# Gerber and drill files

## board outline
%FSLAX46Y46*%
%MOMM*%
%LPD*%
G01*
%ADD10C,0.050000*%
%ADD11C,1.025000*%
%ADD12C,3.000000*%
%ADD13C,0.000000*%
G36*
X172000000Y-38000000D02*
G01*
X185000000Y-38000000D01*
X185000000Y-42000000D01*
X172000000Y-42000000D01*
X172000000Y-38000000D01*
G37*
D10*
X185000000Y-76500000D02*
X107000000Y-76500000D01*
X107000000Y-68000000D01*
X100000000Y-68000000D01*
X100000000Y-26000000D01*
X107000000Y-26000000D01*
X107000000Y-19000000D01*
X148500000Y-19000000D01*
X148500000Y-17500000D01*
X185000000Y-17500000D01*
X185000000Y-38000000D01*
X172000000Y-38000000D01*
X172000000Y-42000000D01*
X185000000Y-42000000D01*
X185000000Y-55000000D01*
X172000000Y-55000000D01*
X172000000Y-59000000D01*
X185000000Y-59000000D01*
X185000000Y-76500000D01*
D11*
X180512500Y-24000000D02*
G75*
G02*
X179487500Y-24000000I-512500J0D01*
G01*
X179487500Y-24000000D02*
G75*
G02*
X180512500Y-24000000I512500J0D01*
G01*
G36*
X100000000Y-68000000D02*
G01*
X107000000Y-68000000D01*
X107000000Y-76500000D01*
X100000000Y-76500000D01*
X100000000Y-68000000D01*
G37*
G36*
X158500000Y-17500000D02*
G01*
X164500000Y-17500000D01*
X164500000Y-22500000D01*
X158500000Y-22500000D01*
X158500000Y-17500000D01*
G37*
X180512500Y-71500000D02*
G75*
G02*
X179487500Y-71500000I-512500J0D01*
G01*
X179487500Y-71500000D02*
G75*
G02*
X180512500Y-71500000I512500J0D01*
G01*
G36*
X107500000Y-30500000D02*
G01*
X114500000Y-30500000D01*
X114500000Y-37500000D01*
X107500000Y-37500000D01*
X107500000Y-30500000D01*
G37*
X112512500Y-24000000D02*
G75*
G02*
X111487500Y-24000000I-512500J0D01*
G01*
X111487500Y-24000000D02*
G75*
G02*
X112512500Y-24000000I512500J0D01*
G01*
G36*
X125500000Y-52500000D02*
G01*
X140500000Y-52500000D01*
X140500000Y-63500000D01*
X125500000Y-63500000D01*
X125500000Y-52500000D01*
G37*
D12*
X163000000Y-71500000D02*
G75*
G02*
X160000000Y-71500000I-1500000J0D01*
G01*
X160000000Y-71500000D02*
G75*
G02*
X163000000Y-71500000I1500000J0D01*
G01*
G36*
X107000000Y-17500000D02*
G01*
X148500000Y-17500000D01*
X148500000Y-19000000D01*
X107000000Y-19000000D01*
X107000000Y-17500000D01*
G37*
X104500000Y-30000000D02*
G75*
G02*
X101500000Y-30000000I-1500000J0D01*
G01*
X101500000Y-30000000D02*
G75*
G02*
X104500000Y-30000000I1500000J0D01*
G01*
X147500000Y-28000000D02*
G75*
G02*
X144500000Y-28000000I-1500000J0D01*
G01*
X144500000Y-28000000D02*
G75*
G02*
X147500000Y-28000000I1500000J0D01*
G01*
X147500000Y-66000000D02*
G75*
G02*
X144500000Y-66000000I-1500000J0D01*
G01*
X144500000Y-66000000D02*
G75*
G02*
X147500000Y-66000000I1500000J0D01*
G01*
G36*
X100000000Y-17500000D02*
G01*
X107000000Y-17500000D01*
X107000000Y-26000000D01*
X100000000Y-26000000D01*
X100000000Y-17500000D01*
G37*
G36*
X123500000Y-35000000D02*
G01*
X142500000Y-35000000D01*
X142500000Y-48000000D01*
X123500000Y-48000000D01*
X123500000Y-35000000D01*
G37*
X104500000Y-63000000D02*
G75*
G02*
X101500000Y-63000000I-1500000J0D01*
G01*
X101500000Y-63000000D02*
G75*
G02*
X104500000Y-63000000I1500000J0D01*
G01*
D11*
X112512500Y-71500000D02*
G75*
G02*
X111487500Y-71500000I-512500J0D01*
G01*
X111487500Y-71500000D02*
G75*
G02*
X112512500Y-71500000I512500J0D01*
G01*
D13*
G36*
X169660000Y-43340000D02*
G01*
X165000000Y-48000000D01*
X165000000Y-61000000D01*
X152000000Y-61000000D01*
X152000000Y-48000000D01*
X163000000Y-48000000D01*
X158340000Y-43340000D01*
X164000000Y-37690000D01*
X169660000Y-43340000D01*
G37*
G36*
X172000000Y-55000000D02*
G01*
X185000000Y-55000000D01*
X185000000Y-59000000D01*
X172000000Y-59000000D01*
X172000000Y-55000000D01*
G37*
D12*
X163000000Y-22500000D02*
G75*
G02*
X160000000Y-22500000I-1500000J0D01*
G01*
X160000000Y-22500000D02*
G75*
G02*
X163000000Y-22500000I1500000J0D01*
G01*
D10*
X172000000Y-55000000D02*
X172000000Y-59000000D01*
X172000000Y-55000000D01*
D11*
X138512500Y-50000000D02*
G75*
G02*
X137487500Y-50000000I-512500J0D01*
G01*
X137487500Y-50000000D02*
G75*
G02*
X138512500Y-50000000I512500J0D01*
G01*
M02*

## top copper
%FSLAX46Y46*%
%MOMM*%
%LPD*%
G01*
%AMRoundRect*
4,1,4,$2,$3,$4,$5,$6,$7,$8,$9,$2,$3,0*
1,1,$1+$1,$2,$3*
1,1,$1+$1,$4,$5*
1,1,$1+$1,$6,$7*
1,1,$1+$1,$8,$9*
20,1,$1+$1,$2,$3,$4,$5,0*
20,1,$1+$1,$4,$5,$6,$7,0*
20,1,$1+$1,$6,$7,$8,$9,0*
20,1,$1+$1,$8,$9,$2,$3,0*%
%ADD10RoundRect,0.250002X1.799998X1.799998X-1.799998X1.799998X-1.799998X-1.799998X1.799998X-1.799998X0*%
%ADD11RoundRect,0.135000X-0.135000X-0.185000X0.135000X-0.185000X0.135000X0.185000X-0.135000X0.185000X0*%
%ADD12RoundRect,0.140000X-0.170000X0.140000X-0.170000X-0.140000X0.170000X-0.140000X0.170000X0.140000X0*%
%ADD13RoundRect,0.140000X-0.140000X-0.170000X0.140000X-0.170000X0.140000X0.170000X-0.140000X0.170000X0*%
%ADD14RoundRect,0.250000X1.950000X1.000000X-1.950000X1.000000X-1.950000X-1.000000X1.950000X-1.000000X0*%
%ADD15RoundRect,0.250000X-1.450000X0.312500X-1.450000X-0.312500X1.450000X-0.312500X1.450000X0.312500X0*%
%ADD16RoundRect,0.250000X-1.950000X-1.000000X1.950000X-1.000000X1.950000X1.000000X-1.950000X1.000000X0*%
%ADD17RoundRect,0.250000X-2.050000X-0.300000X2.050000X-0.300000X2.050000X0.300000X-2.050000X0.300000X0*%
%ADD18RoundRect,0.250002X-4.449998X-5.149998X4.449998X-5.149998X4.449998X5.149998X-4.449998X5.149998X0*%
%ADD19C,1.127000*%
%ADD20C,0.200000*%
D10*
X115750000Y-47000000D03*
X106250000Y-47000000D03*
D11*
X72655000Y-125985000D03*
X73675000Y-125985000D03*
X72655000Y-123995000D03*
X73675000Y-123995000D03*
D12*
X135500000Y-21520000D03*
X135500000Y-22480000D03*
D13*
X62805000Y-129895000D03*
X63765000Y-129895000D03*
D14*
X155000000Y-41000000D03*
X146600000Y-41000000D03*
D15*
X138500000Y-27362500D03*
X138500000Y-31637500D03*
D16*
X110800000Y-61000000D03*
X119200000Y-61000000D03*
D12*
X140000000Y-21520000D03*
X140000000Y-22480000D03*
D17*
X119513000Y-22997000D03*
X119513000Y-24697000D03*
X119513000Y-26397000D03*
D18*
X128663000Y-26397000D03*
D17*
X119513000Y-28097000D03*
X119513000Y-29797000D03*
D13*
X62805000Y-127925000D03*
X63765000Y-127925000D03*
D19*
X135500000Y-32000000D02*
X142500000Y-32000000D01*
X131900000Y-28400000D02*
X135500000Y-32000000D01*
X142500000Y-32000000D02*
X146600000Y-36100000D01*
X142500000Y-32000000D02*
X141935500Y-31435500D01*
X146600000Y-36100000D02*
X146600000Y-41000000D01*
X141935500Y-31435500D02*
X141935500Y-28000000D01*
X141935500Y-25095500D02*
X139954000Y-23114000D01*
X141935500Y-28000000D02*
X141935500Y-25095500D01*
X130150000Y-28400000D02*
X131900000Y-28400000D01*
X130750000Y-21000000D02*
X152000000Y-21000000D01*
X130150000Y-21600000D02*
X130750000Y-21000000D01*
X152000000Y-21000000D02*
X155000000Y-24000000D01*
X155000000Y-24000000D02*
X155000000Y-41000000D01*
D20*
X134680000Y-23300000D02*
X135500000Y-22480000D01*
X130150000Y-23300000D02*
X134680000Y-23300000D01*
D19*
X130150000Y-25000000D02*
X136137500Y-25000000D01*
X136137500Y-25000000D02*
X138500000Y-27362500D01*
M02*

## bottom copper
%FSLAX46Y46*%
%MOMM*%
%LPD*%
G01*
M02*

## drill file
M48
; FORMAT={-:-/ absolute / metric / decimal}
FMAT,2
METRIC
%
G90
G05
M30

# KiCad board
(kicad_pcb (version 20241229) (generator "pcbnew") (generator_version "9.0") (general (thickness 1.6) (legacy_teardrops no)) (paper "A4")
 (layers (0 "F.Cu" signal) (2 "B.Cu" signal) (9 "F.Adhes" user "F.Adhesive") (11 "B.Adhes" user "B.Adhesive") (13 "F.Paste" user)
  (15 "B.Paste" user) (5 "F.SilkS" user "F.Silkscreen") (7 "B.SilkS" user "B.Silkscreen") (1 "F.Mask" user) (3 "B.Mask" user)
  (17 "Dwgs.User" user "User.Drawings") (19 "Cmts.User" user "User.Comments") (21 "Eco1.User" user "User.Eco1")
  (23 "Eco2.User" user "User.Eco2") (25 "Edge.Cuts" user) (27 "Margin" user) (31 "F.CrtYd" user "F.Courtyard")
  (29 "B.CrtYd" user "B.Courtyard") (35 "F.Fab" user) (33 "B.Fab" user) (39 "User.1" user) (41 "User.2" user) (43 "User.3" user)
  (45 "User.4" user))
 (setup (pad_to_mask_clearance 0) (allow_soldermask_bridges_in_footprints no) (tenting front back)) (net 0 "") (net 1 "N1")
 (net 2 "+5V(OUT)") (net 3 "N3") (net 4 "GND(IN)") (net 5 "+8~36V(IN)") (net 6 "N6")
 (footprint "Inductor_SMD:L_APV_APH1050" (layer "F.Cu") (at 111 47 180)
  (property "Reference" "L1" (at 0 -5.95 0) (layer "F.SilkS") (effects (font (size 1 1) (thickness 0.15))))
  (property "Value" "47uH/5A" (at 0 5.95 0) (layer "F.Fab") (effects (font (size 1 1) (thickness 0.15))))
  (pad "1" smd roundrect (at -4.75 0 180) (size 4.1 4.1) (layers "F.Cu" "F.Mask" "F.Paste") (roundrect_rratio 0.060976) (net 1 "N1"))
  (pad "2" smd roundrect (at 4.75 0 180) (size 4.1 4.1) (layers "F.Cu" "F.Mask" "F.Paste") (roundrect_rratio 0.060976) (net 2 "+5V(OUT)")))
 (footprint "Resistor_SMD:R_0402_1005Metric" (layer "F.Cu") (at 73.165 125.985)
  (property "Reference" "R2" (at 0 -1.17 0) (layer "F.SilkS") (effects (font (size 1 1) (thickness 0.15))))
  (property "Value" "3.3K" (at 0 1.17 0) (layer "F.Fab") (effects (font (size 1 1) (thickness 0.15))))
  (pad "1" smd roundrect (at -0.51 0) (size 0.54 0.64) (layers "F.Cu" "F.Mask" "F.Paste") (roundrect_rratio 0.25) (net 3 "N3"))
  (pad "2" smd roundrect (at 0.51 0) (size 0.54 0.64) (layers "F.Cu" "F.Mask" "F.Paste") (roundrect_rratio 0.25) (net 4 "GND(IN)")))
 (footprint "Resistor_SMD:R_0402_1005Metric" (layer "F.Cu") (at 73.165 123.995)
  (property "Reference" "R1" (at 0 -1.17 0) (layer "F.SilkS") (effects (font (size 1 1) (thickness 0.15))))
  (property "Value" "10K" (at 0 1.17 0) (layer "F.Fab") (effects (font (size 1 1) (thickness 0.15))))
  (pad "1" smd roundrect (at -0.51 0) (size 0.54 0.64) (layers "F.Cu" "F.Mask" "F.Paste") (roundrect_rratio 0.25) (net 2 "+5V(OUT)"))
  (pad "2" smd roundrect (at 0.51 0) (size 0.54 0.64) (layers "F.Cu" "F.Mask" "F.Paste") (roundrect_rratio 0.25) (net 3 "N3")))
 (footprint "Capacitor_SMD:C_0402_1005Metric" (layer "F.Cu") (at 135.5 22 -90)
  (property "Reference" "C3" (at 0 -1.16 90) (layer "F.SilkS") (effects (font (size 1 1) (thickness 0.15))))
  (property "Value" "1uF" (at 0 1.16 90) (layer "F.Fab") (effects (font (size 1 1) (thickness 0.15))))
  (pad "1" smd roundrect (at -0.48 0 270) (size 0.56 0.62) (layers "F.Cu" "F.Mask" "F.Paste") (roundrect_rratio 0.25) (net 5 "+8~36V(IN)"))
  (pad "2" smd roundrect (at 0.48 0 270) (size 0.56 0.62) (layers "F.Cu" "F.Mask" "F.Paste") (roundrect_rratio 0.25) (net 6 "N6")))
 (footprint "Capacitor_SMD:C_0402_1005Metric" (layer "F.Cu") (at 63.285 129.895)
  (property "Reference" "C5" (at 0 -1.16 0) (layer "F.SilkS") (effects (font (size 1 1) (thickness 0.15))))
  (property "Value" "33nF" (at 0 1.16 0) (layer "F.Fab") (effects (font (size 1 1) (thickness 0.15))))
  (pad "1" smd roundrect (at -0.48 0) (size 0.56 0.62) (layers "F.Cu" "F.Mask" "F.Paste") (roundrect_rratio 0.25) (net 2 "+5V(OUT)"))
  (pad "2" smd roundrect (at 0.48 0) (size 0.56 0.62) (layers "F.Cu" "F.Mask" "F.Paste") (roundrect_rratio 0.25) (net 3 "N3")))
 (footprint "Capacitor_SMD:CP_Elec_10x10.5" (layer "F.Cu") (at 150.8 41 180)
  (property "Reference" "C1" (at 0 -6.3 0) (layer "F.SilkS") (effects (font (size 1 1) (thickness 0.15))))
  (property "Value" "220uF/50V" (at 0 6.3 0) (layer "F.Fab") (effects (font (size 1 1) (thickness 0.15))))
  (pad "1" smd roundrect (at -4.2 0 180) (size 4.4 2.5) (layers "F.Cu" "F.Mask" "F.Paste") (roundrect_rratio 0.1) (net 5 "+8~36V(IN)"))
  (pad "2" smd roundrect (at 4.2 0 180) (size 4.4 2.5) (layers "F.Cu" "F.Mask" "F.Paste") (roundrect_rratio 0.1) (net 4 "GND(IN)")))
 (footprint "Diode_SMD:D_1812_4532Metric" (layer "F.Cu") (at 138.5 29.5 -90)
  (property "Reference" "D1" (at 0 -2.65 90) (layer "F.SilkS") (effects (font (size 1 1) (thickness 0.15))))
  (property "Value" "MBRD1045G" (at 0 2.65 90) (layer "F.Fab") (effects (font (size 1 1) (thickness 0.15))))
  (pad "1" smd roundrect (at -2.1375 0 270) (size 1.125 3.4) (layers "F.Cu" "F.Mask" "F.Paste") (roundrect_rratio 0.222222) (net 1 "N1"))
  (pad "2" smd roundrect (at 2.1375 0 270) (size 1.125 3.4) (layers "F.Cu" "F.Mask" "F.Paste") (roundrect_rratio 0.222222) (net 4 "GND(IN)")))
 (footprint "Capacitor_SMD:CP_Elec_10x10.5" (layer "F.Cu") (at 115 61)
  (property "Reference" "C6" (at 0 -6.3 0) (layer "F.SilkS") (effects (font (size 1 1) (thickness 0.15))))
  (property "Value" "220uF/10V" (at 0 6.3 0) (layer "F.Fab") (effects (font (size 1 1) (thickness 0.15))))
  (pad "1" smd roundrect (at -4.2 0) (size 4.4 2.5) (layers "F.Cu" "F.Mask" "F.Paste") (roundrect_rratio 0.1) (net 2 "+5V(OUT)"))
  (pad "2" smd roundrect (at 4.2 0) (size 4.4 2.5) (layers "F.Cu" "F.Mask" "F.Paste") (roundrect_rratio 0.1) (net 4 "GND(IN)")))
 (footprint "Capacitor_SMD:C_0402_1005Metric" (layer "F.Cu") (at 140 22 -90)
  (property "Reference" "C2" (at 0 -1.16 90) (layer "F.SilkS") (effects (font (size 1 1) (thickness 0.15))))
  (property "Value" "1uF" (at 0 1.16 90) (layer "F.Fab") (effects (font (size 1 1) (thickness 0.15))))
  (pad "1" smd roundrect (at -0.48 0 270) (size 0.56 0.62) (layers "F.Cu" "F.Mask" "F.Paste") (roundrect_rratio 0.25) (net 5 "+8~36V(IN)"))
  (pad "2" smd roundrect (at 0.48 0 270) (size 0.56 0.62) (layers "F.Cu" "F.Mask" "F.Paste") (roundrect_rratio 0.25) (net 4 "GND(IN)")))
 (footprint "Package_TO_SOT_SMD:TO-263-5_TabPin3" (layer "F.Cu") (at 127.163 26.397)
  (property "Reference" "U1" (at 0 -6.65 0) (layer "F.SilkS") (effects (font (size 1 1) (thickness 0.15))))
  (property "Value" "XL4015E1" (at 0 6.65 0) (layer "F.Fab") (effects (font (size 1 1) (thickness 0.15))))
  (pad "" smd roundrect (at -0.925 -2.775) (size 4.55 5.25) (layers "F.Paste") (roundrect_rratio 0.054945))
  (pad "" smd roundrect (at -0.925 2.775) (size 4.55 5.25) (layers "F.Paste") (roundrect_rratio 0.054945))
  (pad "" smd roundrect (at 3.925 -2.775) (size 4.55 5.25) (layers "F.Paste") (roundrect_rratio 0.054945))
  (pad "" smd roundrect (at 3.925 2.775) (size 4.55 5.25) (layers "F.Paste") (roundrect_rratio 0.054945))
  (pad "1" smd roundrect (at -7.65 -3.4) (size 4.6 1.1) (layers "F.Cu" "F.Mask" "F.Paste") (roundrect_rratio 0.227273) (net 4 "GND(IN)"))
  (pad "2" smd roundrect (at -7.65 -1.7) (size 4.6 1.1) (layers "F.Cu" "F.Mask" "F.Paste") (roundrect_rratio 0.227273) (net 3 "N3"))
  (pad "3" smd roundrect (at -7.65 0) (size 4.6 1.1) (layers "F.Cu" "F.Mask" "F.Paste") (roundrect_rratio 0.227273) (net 1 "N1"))
  (pad "3" smd roundrect (at 1.5 0) (size 9.4 10.8) (layers "F.Cu" "F.Mask") (roundrect_rratio 0.026596) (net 1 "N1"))
  (pad "4" smd roundrect (at -7.65 1.7) (size 4.6 1.1) (layers "F.Cu" "F.Mask" "F.Paste") (roundrect_rratio 0.227273) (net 6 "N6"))
  (pad "5" smd roundrect (at -7.65 3.4) (size 4.6 1.1) (layers "F.Cu" "F.Mask" "F.Paste") (roundrect_rratio 0.227273) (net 5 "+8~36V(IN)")))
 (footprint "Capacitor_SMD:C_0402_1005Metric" (layer "F.Cu") (at 63.285 127.925)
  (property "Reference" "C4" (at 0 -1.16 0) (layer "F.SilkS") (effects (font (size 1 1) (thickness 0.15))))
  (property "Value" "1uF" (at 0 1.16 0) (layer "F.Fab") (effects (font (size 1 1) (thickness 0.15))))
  (pad "1" smd roundrect (at -0.48 0) (size 0.56 0.62) (layers "F.Cu" "F.Mask" "F.Paste") (roundrect_rratio 0.25) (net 2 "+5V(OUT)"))
  (pad "2" smd roundrect (at 0.48 0) (size 0.56 0.62) (layers "F.Cu" "F.Mask" "F.Paste") (roundrect_rratio 0.25) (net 4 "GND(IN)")))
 (gr_rect (start 172 38) (end 185 42) (stroke (width 0) (type solid)) (fill yes) (layer "Edge.Cuts"))
 (gr_poly
  (pts (xy 185 76.5) (xy 107 76.5) (xy 107 68) (xy 100 68) (xy 100 26) (xy 107 26) (xy 107 19) (xy 148.5 19) (xy 148.5 17.5) (xy 185 17.5)
   (xy 185 38) (xy 172 38) (xy 172 42) (xy 185 42) (xy 185 55) (xy 172 55) (xy 172 59) (xy 185 59))
  (stroke (width 0.05) (type solid)) (fill no) (layer "Edge.Cuts"))
 (gr_circle (center 180 24) (end 181.025 24) (stroke (width 0) (type default)) (fill yes) (layer "Edge.Cuts"))
 (gr_rect (start 100 68) (end 107 76.5) (stroke (width 0) (type default)) (fill yes) (layer "Edge.Cuts"))
 (gr_rect (start 158.5 17.5) (end 164.5 22.5) (stroke (width 0) (type solid)) (fill yes) (layer "Edge.Cuts"))
 (gr_circle (center 180 71.5) (end 181.025 71.5) (stroke (width 0) (type default)) (fill yes) (layer "Edge.Cuts"))
 (gr_rect (start 107.5 30.5) (end 114.5 37.5) (stroke (width 0) (type solid)) (fill yes) (layer "Edge.Cuts"))
 (gr_circle (center 112 24) (end 113.025 24) (stroke (width 0) (type default)) (fill yes) (layer "Edge.Cuts"))
 (gr_rect (start 125.5 52.5) (end 140.5 63.5) (stroke (width 0) (type solid)) (fill yes) (layer "Edge.Cuts"))
 (gr_circle (center 161.5 71.5) (end 164.5 71.5) (stroke (width 0) (type solid)) (fill yes) (layer "Edge.Cuts"))
 (gr_rect (start 107 17.5) (end 148.5 19) (stroke (width 0) (type default)) (fill yes) (layer "Edge.Cuts"))
 (gr_circle (center 103 30) (end 106 30) (stroke (width 0) (type solid)) (fill yes) (layer "Edge.Cuts"))
 (gr_circle (center 146 28) (end 149 28) (stroke (width 0) (type solid)) (fill yes) (layer "Edge.Cuts"))
 (gr_circle (center 146 66) (end 149 66) (stroke (width 0) (type solid)) (fill yes) (layer "Edge.Cuts"))
 (gr_rect (start 100 17.5) (end 107 26) (stroke (width 0) (type default)) (fill yes) (layer "Edge.Cuts"))
 (gr_rect (start 123.5 35) (end 142.5 48) (stroke (width 0) (type solid)) (fill yes) (layer "Edge.Cuts"))
 (gr_circle (center 103 63) (end 106 63) (stroke (width 0) (type solid)) (fill yes) (layer "Edge.Cuts"))
 (gr_circle (center 112 71.5) (end 113.025 71.5) (stroke (width 0) (type default)) (fill yes) (layer "Edge.Cuts"))
 (gr_poly
  (pts (xy 152 61) (xy 152 48) (xy 163 48) (xy 158.34 43.34) (xy 164 37.69) (xy 169.66 43.34) (xy 165 48) (xy 165 61))
  (stroke (width 0) (type solid)) (fill yes) (layer "Edge.Cuts"))
 (gr_rect (start 172 55) (end 185 59) (stroke (width 0) (type solid)) (fill yes) (layer "Edge.Cuts"))
 (gr_circle (center 161.5 22.5) (end 164.5 22.5) (stroke (width 0) (type solid)) (fill yes) (layer "Edge.Cuts"))
 (gr_rect (start 172 55) (end 172 59) (stroke (width 0.05) (type default)) (fill no) (layer "Edge.Cuts"))
 (gr_circle (center 138 50) (end 139.025 50) (stroke (width 0) (type default)) (fill yes) (layer "Edge.Cuts"))
 (segment (start 135.5 32) (end 142.5 32) (width 1.127) (layer "F.Cu") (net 4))
 (segment (start 131.9 28.4) (end 135.5 32) (width 1.127) (layer "F.Cu") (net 4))
 (segment (start 142.5 32) (end 146.6 36.1) (width 1.127) (layer "F.Cu") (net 4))
 (segment (start 142.5 32) (end 141.9355 31.4355) (width 1.127) (layer "F.Cu") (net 4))
 (segment (start 146.6 36.1) (end 146.6 41) (width 1.127) (layer "F.Cu") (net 4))
 (segment (start 141.9355 31.4355) (end 141.9355 28) (width 1.127) (layer "F.Cu") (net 4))
 (segment (start 141.9355 25.0955) (end 139.954 23.114) (width 1.127) (layer "F.Cu") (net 4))
 (segment (start 141.9355 28) (end 141.9355 25.0955) (width 1.127) (layer "F.Cu") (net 4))
 (segment (start 130.15 28.4) (end 131.9 28.4) (width 1.127) (layer "F.Cu") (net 4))
 (segment (start 130.75 21) (end 152 21) (width 1.127) (layer "F.Cu") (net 5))
 (segment (start 130.15 21.6) (end 130.75 21) (width 1.127) (layer "F.Cu") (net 5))
 (segment (start 152 21) (end 155 24) (width 1.127) (layer "F.Cu") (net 5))
 (segment (start 155 24) (end 155 41) (width 1.127) (layer "F.Cu") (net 5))
 (segment (start 134.68 23.3) (end 135.5 22.48) (width 0.2) (layer "F.Cu") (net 6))
 (segment (start 130.15 23.3) (end 134.68 23.3) (width 0.2) (layer "F.Cu") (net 6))
 (segment (start 130.15 25) (end 136.1375 25) (width 1.127) (layer "F.Cu") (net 1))
 (segment (start 136.1375 25) (end 138.5 27.3625) (width 1.127) (layer "F.Cu") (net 1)))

